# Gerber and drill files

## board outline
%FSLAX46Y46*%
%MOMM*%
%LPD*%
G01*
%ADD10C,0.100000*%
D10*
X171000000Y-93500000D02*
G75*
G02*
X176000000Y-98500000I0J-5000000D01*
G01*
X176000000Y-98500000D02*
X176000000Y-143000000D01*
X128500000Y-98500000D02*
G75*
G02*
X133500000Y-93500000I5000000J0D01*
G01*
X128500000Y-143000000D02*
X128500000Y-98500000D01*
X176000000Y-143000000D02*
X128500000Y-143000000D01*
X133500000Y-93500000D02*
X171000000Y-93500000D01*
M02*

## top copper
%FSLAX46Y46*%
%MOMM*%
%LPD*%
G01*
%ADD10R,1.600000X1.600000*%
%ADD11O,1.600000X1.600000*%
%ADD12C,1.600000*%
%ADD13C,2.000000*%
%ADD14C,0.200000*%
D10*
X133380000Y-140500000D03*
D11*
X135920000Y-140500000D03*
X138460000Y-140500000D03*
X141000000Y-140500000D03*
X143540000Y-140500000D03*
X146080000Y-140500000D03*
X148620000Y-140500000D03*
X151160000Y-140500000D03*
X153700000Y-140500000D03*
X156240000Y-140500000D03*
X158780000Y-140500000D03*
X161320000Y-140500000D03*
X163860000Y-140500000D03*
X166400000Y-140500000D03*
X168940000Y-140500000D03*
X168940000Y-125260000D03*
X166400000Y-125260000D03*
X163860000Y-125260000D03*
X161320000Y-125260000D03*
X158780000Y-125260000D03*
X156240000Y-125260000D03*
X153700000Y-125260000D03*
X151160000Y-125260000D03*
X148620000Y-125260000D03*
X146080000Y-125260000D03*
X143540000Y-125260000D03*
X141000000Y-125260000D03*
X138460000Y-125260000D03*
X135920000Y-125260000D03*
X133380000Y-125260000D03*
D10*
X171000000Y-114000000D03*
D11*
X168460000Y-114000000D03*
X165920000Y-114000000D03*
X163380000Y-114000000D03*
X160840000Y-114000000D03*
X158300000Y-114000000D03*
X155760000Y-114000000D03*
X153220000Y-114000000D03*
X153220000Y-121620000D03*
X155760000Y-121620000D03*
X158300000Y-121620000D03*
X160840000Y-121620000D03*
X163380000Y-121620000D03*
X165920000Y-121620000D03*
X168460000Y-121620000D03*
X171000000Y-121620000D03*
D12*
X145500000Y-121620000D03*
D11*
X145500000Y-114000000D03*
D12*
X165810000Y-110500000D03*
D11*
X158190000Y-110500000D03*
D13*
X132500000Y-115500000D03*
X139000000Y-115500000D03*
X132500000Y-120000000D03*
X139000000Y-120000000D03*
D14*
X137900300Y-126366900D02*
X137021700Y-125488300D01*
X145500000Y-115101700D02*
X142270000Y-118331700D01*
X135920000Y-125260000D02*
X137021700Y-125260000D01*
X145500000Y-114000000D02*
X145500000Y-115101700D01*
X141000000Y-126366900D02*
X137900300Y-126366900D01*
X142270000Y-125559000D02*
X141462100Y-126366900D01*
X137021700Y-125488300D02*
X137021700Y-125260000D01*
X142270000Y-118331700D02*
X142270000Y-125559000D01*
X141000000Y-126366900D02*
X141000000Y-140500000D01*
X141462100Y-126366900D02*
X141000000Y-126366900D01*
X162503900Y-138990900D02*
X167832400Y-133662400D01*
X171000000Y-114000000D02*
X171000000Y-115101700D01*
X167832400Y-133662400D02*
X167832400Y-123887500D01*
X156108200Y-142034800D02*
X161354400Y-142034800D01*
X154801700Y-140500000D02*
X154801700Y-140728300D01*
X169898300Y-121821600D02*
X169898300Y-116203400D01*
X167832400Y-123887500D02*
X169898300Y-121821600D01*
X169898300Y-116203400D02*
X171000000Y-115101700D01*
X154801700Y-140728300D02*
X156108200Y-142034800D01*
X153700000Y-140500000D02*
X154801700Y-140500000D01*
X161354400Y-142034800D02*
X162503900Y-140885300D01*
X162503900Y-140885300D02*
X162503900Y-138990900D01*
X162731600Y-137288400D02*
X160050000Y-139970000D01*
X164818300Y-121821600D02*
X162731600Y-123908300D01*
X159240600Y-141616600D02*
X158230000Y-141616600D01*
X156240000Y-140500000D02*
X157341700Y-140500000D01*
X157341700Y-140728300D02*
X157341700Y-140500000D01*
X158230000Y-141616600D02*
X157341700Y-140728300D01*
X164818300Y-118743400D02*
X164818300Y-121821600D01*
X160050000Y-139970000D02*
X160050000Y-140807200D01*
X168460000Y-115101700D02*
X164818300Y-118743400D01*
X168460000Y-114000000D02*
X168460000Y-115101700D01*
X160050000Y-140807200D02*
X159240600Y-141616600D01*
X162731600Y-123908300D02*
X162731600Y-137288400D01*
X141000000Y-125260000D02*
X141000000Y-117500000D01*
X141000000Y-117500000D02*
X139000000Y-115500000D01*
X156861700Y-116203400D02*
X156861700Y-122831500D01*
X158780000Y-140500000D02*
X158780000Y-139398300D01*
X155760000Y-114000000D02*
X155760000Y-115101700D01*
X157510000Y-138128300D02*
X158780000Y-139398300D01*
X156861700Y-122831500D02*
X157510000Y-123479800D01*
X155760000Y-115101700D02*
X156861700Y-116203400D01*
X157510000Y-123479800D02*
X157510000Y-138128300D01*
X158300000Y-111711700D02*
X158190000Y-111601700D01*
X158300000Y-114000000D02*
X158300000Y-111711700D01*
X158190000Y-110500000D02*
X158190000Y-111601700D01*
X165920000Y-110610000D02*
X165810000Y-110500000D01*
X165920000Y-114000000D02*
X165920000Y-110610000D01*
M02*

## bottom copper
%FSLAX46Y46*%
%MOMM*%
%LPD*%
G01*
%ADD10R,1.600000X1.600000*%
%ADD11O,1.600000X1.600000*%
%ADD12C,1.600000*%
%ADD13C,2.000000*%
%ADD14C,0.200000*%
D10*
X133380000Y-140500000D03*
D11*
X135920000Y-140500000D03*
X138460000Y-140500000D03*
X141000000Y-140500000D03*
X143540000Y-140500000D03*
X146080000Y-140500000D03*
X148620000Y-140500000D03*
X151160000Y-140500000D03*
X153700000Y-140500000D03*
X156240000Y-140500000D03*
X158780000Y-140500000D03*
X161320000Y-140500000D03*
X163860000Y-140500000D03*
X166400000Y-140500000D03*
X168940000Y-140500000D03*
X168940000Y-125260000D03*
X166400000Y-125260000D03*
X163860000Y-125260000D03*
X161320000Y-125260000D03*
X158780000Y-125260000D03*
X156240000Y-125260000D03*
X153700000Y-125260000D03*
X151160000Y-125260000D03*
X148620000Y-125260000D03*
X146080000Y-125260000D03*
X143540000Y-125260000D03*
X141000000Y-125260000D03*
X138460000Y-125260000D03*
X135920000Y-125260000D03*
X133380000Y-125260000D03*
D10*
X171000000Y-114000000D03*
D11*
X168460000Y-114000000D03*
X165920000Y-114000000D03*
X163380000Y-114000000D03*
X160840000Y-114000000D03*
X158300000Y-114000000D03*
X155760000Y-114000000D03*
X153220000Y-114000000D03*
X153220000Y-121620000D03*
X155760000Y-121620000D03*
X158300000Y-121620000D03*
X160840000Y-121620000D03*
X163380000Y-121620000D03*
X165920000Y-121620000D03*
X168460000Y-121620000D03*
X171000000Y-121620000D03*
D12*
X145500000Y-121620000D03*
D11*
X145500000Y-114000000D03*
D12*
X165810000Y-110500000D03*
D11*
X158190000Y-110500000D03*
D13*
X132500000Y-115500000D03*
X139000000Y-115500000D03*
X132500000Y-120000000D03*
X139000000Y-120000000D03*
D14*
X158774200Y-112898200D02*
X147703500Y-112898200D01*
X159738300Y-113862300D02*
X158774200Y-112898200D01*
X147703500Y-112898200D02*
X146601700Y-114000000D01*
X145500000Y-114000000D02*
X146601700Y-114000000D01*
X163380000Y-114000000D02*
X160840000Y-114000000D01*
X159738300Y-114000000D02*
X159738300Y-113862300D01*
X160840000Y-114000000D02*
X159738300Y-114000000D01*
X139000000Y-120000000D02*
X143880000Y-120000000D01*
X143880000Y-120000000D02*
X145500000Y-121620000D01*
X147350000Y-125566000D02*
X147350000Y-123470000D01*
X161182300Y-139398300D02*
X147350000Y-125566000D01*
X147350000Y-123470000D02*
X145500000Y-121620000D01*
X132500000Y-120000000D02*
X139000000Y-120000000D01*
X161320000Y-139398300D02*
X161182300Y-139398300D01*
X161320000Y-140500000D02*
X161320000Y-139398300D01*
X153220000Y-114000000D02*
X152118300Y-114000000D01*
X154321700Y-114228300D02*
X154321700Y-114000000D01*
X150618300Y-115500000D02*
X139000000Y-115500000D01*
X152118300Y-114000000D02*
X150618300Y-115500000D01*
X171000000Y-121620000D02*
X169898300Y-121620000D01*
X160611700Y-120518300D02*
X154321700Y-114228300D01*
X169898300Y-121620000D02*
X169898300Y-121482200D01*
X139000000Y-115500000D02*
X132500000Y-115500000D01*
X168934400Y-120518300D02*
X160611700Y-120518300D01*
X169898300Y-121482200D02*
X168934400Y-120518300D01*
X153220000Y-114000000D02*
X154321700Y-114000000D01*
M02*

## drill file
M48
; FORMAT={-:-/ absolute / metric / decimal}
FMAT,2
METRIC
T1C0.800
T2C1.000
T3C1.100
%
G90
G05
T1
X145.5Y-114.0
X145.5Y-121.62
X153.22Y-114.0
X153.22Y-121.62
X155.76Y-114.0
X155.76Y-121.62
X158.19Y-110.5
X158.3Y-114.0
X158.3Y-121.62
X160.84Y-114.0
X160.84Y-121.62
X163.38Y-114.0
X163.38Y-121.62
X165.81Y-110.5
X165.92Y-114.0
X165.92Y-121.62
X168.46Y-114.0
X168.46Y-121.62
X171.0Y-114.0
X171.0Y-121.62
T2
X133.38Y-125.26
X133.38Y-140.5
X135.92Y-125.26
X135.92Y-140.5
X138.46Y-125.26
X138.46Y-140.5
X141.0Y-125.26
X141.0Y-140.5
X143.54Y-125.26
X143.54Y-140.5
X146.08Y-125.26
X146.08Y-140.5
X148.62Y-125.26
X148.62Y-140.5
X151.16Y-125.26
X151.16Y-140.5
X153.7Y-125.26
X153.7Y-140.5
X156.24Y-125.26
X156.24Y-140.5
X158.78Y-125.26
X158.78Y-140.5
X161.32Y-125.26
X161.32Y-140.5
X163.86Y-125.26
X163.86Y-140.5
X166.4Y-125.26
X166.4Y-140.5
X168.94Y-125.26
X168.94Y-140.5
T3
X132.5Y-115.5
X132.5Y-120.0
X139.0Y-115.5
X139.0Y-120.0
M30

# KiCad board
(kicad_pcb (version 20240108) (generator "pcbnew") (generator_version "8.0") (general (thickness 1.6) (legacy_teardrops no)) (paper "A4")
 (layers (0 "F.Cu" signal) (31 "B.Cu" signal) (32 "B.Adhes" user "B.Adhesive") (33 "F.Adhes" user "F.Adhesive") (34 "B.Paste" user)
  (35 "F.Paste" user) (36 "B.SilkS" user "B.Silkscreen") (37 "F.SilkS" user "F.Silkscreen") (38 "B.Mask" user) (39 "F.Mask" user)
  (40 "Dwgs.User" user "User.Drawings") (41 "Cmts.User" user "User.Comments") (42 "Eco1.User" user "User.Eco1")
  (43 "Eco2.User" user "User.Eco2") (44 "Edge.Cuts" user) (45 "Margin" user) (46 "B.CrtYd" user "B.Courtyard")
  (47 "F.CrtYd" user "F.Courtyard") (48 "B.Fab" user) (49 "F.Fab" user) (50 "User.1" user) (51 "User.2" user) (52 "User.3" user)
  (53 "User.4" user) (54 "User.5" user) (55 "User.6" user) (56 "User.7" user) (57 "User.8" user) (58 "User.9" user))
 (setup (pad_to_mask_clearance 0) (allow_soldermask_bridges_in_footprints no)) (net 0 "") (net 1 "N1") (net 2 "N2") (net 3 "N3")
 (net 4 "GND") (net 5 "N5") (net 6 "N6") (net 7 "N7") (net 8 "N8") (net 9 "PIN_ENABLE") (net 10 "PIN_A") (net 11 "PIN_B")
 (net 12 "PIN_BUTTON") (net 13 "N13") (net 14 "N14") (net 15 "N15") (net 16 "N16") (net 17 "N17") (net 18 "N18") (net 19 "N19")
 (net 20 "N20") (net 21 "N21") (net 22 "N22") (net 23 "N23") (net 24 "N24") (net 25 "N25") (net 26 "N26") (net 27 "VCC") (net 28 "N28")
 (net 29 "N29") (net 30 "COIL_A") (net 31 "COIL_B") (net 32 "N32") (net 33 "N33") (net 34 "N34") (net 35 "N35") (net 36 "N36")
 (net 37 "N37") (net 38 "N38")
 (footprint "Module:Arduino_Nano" (layer "F.Cu") (at 133.38 140.5 90)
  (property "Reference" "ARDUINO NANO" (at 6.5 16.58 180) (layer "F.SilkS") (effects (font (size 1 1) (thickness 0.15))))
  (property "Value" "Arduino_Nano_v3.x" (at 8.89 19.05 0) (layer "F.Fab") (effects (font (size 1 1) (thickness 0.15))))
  (pad "1" thru_hole rect (at 0 0 90) (size 1.6 1.6) (drill 1) (layers "*.Cu" "*.Mask") (remove_unused_layers no) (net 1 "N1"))
  (pad "2" thru_hole oval (at 0 2.54 90) (size 1.6 1.6) (drill 1) (layers "*.Cu" "*.Mask") (remove_unused_layers no) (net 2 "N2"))
  (pad "3" thru_hole oval (at 0 5.08 90) (size 1.6 1.6) (drill 1) (layers "*.Cu" "*.Mask") (remove_unused_layers no) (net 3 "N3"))
  (pad "4" thru_hole oval (at 0 7.62 90) (size 1.6 1.6) (drill 1) (layers "*.Cu" "*.Mask") (remove_unused_layers no) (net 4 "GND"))
  (pad "5" thru_hole oval (at 0 10.16 90) (size 1.6 1.6) (drill 1) (layers "*.Cu" "*.Mask") (remove_unused_layers no) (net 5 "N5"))
  (pad "6" thru_hole oval (at 0 12.7 90) (size 1.6 1.6) (drill 1) (layers "*.Cu" "*.Mask") (remove_unused_layers no) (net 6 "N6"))
  (pad "7" thru_hole oval (at 0 15.24 90) (size 1.6 1.6) (drill 1) (layers "*.Cu" "*.Mask") (remove_unused_layers no) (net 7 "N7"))
  (pad "8" thru_hole oval (at 0 17.78 90) (size 1.6 1.6) (drill 1) (layers "*.Cu" "*.Mask") (remove_unused_layers no) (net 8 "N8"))
  (pad "9" thru_hole oval (at 0 20.32 90) (size 1.6 1.6) (drill 1) (layers "*.Cu" "*.Mask") (remove_unused_layers no) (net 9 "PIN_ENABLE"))
  (pad "10" thru_hole oval (at 0 22.86 90) (size 1.6 1.6) (drill 1) (layers "*.Cu" "*.Mask") (remove_unused_layers no) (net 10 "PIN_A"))
  (pad "11" thru_hole oval (at 0 25.4 90) (size 1.6 1.6) (drill 1) (layers "*.Cu" "*.Mask") (remove_unused_layers no) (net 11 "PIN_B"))
  (pad "12" thru_hole oval (at 0 27.94 90) (size 1.6 1.6) (drill 1) (layers "*.Cu" "*.Mask") (remove_unused_layers no) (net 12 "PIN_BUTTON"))
  (pad "13" thru_hole oval (at 0 30.48 90) (size 1.6 1.6) (drill 1) (layers "*.Cu" "*.Mask") (remove_unused_layers no) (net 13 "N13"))
  (pad "14" thru_hole oval (at 0 33.02 90) (size 1.6 1.6) (drill 1) (layers "*.Cu" "*.Mask") (remove_unused_layers no) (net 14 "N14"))
  (pad "15" thru_hole oval (at 0 35.56 90) (size 1.6 1.6) (drill 1) (layers "*.Cu" "*.Mask") (remove_unused_layers no) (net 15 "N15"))
  (pad "16" thru_hole oval (at 15.24 35.56 90) (size 1.6 1.6) (drill 1) (layers "*.Cu" "*.Mask") (remove_unused_layers no) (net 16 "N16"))
  (pad "17" thru_hole oval (at 15.24 33.02 90) (size 1.6 1.6) (drill 1) (layers "*.Cu" "*.Mask") (remove_unused_layers no) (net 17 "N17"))
  (pad "18" thru_hole oval (at 15.24 30.48 90) (size 1.6 1.6) (drill 1) (layers "*.Cu" "*.Mask") (remove_unused_layers no) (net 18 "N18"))
  (pad "19" thru_hole oval (at 15.24 27.94 90) (size 1.6 1.6) (drill 1) (layers "*.Cu" "*.Mask") (remove_unused_layers no) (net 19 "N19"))
  (pad "20" thru_hole oval (at 15.24 25.4 90) (size 1.6 1.6) (drill 1) (layers "*.Cu" "*.Mask") (remove_unused_layers no) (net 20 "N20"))
  (pad "21" thru_hole oval (at 15.24 22.86 90) (size 1.6 1.6) (drill 1) (layers "*.Cu" "*.Mask") (remove_unused_layers no) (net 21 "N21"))
  (pad "22" thru_hole oval (at 15.24 20.32 90) (size 1.6 1.6) (drill 1) (layers "*.Cu" "*.Mask") (remove_unused_layers no) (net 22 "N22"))
  (pad "23" thru_hole oval (at 15.24 17.78 90) (size 1.6 1.6) (drill 1) (layers "*.Cu" "*.Mask") (remove_unused_layers no) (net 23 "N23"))
  (pad "24" thru_hole oval (at 15.24 15.24 90) (size 1.6 1.6) (drill 1) (layers "*.Cu" "*.Mask") (remove_unused_layers no) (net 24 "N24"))
  (pad "25" thru_hole oval (at 15.24 12.7 90) (size 1.6 1.6) (drill 1) (layers "*.Cu" "*.Mask") (remove_unused_layers no) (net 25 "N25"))
  (pad "26" thru_hole oval (at 15.24 10.16 90) (size 1.6 1.6) (drill 1) (layers "*.Cu" "*.Mask") (remove_unused_layers no) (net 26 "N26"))
  (pad "27" thru_hole oval (at 15.24 7.62 90) (size 1.6 1.6) (drill 1) (layers "*.Cu" "*.Mask") (remove_unused_layers no) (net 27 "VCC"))
  (pad "28" thru_hole oval (at 15.24 5.08 90) (size 1.6 1.6) (drill 1) (layers "*.Cu" "*.Mask") (remove_unused_layers no) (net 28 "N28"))
  (pad "29" thru_hole oval (at 15.24 2.54 90) (size 1.6 1.6) (drill 1) (layers "*.Cu" "*.Mask") (remove_unused_layers no) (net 4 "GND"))
  (pad "30" thru_hole oval (at 15.24 0 90) (size 1.6 1.6) (drill 1) (layers "*.Cu" "*.Mask") (remove_unused_layers no) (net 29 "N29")))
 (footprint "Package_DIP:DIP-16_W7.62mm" (layer "F.Cu") (at 171 114 -90)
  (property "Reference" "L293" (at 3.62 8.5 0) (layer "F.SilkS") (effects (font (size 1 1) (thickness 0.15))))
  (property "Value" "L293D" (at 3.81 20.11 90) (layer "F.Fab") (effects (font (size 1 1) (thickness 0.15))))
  (pad "1" thru_hole rect (at 0 0 270) (size 1.6 1.6) (drill 0.8) (layers "*.Cu" "*.Mask") (remove_unused_layers no) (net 9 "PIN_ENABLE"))
  (pad "2" thru_hole oval (at 0 2.54 270) (size 1.6 1.6) (drill 0.8) (layers "*.Cu" "*.Mask") (remove_unused_layers no) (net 10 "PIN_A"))
  (pad "3" thru_hole oval (at 0 5.08 270) (size 1.6 1.6) (drill 0.8) (layers "*.Cu" "*.Mask") (remove_unused_layers no) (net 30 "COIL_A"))
  (pad "4" thru_hole oval (at 0 7.62 270) (size 1.6 1.6) (drill 0.8) (layers "*.Cu" "*.Mask") (remove_unused_layers no) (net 4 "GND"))
  (pad "5" thru_hole oval (at 0 10.16 270) (size 1.6 1.6) (drill 0.8) (layers "*.Cu" "*.Mask") (remove_unused_layers no) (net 4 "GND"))
  (pad "6" thru_hole oval (at 0 12.7 270) (size 1.6 1.6) (drill 0.8) (layers "*.Cu" "*.Mask") (remove_unused_layers no) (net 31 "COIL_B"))
  (pad "7" thru_hole oval (at 0 15.24 270) (size 1.6 1.6) (drill 0.8) (layers "*.Cu" "*.Mask") (remove_unused_layers no) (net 11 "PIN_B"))
  (pad "8" thru_hole oval (at 0 17.78 270) (size 1.6 1.6) (drill 0.8) (layers "*.Cu" "*.Mask") (remove_unused_layers no) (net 27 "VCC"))
  (pad "9" thru_hole oval (at 7.62 17.78 270) (size 1.6 1.6) (drill 0.8) (layers "*.Cu" "*.Mask") (remove_unused_layers no) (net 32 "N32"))
  (pad "10" thru_hole oval (at 7.62 15.24 270) (size 1.6 1.6) (drill 0.8) (layers "*.Cu" "*.Mask") (remove_unused_layers no) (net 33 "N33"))
  (pad "11" thru_hole oval (at 7.62 12.7 270) (size 1.6 1.6) (drill 0.8) (layers "*.Cu" "*.Mask") (remove_unused_layers no) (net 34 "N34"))
  (pad "12" thru_hole oval (at 7.62 10.16 270) (size 1.6 1.6) (drill 0.8) (layers "*.Cu" "*.Mask") (remove_unused_layers no) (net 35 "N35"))
  (pad "13" thru_hole oval (at 7.62 7.62 270) (size 1.6 1.6) (drill 0.8) (layers "*.Cu" "*.Mask") (remove_unused_layers no) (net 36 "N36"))
  (pad "14" thru_hole oval (at 7.62 5.08 270) (size 1.6 1.6) (drill 0.8) (layers "*.Cu" "*.Mask") (remove_unused_layers no) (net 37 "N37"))
  (pad "15" thru_hole oval (at 7.62 2.54 270) (size 1.6 1.6) (drill 0.8) (layers "*.Cu" "*.Mask") (remove_unused_layers no) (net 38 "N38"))
  (pad "16" thru_hole oval (at 7.62 0 270) (size 1.6 1.6) (drill 0.8) (layers "*.Cu" "*.Mask") (remove_unused_layers no) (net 27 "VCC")))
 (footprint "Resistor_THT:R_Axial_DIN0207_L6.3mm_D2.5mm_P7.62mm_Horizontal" (layer "F.Cu") (at 145.5 121.62 90)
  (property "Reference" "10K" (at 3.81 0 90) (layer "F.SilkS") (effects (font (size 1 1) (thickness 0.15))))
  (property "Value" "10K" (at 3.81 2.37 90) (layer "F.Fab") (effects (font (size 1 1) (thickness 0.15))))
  (pad "1" thru_hole circle (at 0 0 90) (size 1.6 1.6) (drill 0.8) (layers "*.Cu" "*.Mask") (remove_unused_layers no) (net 12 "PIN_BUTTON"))
  (pad "2" thru_hole oval (at 7.62 0 90) (size 1.6 1.6) (drill 0.8) (layers "*.Cu" "*.Mask") (remove_unused_layers no) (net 4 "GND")))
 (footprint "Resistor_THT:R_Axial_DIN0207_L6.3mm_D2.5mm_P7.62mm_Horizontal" (layer "F.Cu") (at 165.81 110.5 180)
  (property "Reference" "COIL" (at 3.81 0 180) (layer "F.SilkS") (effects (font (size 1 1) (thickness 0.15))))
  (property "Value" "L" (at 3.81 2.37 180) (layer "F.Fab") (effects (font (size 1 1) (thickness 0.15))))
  (pad "1" thru_hole circle (at 0 0 180) (size 1.6 1.6) (drill 0.8) (layers "*.Cu" "*.Mask") (remove_unused_layers no) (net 30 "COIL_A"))
  (pad "2" thru_hole oval (at 7.62 0 180) (size 1.6 1.6) (drill 0.8) (layers "*.Cu" "*.Mask") (remove_unused_layers no) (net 31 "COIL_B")))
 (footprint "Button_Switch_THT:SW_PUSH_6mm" (layer "F.Cu") (at 132.5 115.5)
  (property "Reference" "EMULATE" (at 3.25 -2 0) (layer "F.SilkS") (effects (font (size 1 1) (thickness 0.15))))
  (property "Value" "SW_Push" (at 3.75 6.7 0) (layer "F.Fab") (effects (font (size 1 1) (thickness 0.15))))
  (pad "1" thru_hole circle (at 0 0 90) (size 2 2) (drill 1.1) (layers "*.Cu" "*.Mask") (remove_unused_layers no) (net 27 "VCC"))
  (pad "1" thru_hole circle (at 6.5 0 90) (size 2 2) (drill 1.1) (layers "*.Cu" "*.Mask") (remove_unused_layers no) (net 27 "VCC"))
  (pad "2" thru_hole circle (at 0 4.5 90) (size 2 2) (drill 1.1) (layers "*.Cu" "*.Mask") (remove_unused_layers no) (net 12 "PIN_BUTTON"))
  (pad "2" thru_hole circle (at 6.5 4.5 90) (size 2 2) (drill 1.1) (layers "*.Cu" "*.Mask") (remove_unused_layers no) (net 12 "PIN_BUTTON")))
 (gr_arc (start 171 93.5) (mid 174.535534 94.964466) (end 176 98.5) (stroke (width 0.1) (type default)) (layer "Edge.Cuts"))
 (gr_line (start 176 98.5) (end 176 143) (stroke (width 0.1) (type default)) (layer "Edge.Cuts"))
 (gr_arc (start 128.5 98.5) (mid 129.964466 94.964466) (end 133.5 93.5) (stroke (width 0.1) (type default)) (layer "Edge.Cuts"))
 (gr_line (start 128.5 143) (end 128.5 98.5) (stroke (width 0.1) (type default)) (layer "Edge.Cuts"))
 (gr_line (start 176 143) (end 128.5 143) (stroke (width 0.1) (type default)) (layer "Edge.Cuts"))
 (gr_line (start 133.5 93.5) (end 171 93.5) (stroke (width 0.1) (type default)) (layer "Edge.Cuts"))
 (segment (start 137.9003 126.3669) (end 137.0217 125.4883) (width 0.2) (layer "F.Cu") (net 4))
 (segment (start 145.5 115.1017) (end 142.27 118.3317) (width 0.2) (layer "F.Cu") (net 4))
 (segment (start 135.92 125.26) (end 137.0217 125.26) (width 0.2) (layer "F.Cu") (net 4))
 (segment (start 145.5 114) (end 145.5 115.1017) (width 0.2) (layer "F.Cu") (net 4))
 (segment (start 141 126.3669) (end 137.9003 126.3669) (width 0.2) (layer "F.Cu") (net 4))
 (segment (start 142.27 125.559) (end 141.4621 126.3669) (width 0.2) (layer "F.Cu") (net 4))
 (segment (start 137.0217 125.4883) (end 137.0217 125.26) (width 0.2) (layer "F.Cu") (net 4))
 (segment (start 142.27 118.3317) (end 142.27 125.559) (width 0.2) (layer "F.Cu") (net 4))
 (segment (start 141 126.3669) (end 141 140.5) (width 0.2) (layer "F.Cu") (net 4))
 (segment (start 141.4621 126.3669) (end 141 126.3669) (width 0.2) (layer "F.Cu") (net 4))
 (segment (start 158.7742 112.8982) (end 147.7035 112.8982) (width 0.2) (layer "B.Cu") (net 4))
 (segment (start 159.7383 113.8623) (end 158.7742 112.8982) (width 0.2) (layer "B.Cu") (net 4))
 (segment (start 147.7035 112.8982) (end 146.6017 114) (width 0.2) (layer "B.Cu") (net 4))
 (segment (start 145.5 114) (end 146.6017 114) (width 0.2) (layer "B.Cu") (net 4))
 (segment (start 163.38 114) (end 160.84 114) (width 0.2) (layer "B.Cu") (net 4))
 (segment (start 159.7383 114) (end 159.7383 113.8623) (width 0.2) (layer "B.Cu") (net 4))
 (segment (start 160.84 114) (end 159.7383 114) (width 0.2) (layer "B.Cu") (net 4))
 (segment (start 139 120) (end 143.88 120) (width 0.2) (layer "B.Cu") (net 12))
 (segment (start 143.88 120) (end 145.5 121.62) (width 0.2) (layer "B.Cu") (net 12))
 (segment (start 147.35 125.566) (end 147.35 123.47) (width 0.2) (layer "B.Cu") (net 12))
 (segment (start 161.1823 139.3983) (end 147.35 125.566) (width 0.2) (layer "B.Cu") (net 12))
 (segment (start 147.35 123.47) (end 145.5 121.62) (width 0.2) (layer "B.Cu") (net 12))
 (segment (start 132.5 120) (end 139 120) (width 0.2) (layer "B.Cu") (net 12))
 (segment (start 161.32 139.3983) (end 161.1823 139.3983) (width 0.2) (layer "B.Cu") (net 12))
 (segment (start 161.32 140.5) (end 161.32 139.3983) (width 0.2) (layer "B.Cu") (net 12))
 (segment (start 162.5039 138.9909) (end 167.8324 133.6624) (width 0.2) (layer "F.Cu") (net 9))
 (segment (start 171 114) (end 171 115.1017) (width 0.2) (layer "F.Cu") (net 9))
 (segment (start 167.8324 133.6624) (end 167.8324 123.8875) (width 0.2) (layer "F.Cu") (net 9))
 (segment (start 156.1082 142.0348) (end 161.3544 142.0348) (width 0.2) (layer "F.Cu") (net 9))
 (segment (start 154.8017 140.5) (end 154.8017 140.7283) (width 0.2) (layer "F.Cu") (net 9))
 (segment (start 169.8983 121.8216) (end 169.8983 116.2034) (width 0.2) (layer "F.Cu") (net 9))
 (segment (start 167.8324 123.8875) (end 169.8983 121.8216) (width 0.2) (layer "F.Cu") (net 9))
 (segment (start 169.8983 116.2034) (end 171 115.1017) (width 0.2) (layer "F.Cu") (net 9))
 (segment (start 154.8017 140.7283) (end 156.1082 142.0348) (width 0.2) (layer "F.Cu") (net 9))
 (segment (start 153.7 140.5) (end 154.8017 140.5) (width 0.2) (layer "F.Cu") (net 9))
 (segment (start 161.3544 142.0348) (end 162.5039 140.8853) (width 0.2) (layer "F.Cu") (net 9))
 (segment (start 162.5039 140.8853) (end 162.5039 138.9909) (width 0.2) (layer "F.Cu") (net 9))
 (segment (start 162.7316 137.2884) (end 160.05 139.97) (width 0.2) (layer "F.Cu") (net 10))
 (segment (start 164.8183 121.8216) (end 162.7316 123.9083) (width 0.2) (layer "F.Cu") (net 10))
 (segment (start 159.2406 141.6166) (end 158.23 141.6166) (width 0.2) (layer "F.Cu") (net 10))
 (segment (start 156.24 140.5) (end 157.3417 140.5) (width 0.2) (layer "F.Cu") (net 10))
 (segment (start 157.3417 140.7283) (end 157.3417 140.5) (width 0.2) (layer "F.Cu") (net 10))
 (segment (start 158.23 141.6166) (end 157.3417 140.7283) (width 0.2) (layer "F.Cu") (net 10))
 (segment (start 164.8183 118.7434) (end 164.8183 121.8216) (width 0.2) (layer "F.Cu") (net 10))
 (segment (start 160.05 139.97) (end 160.05 140.8072) (width 0.2) (layer "F.Cu") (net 10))
 (segment (start 168.46 115.1017) (end 164.8183 118.7434) (width 0.2) (layer "F.Cu") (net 10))
 (segment (start 168.46 114) (end 168.46 115.1017) (width 0.2) (layer "F.Cu") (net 10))
 (segment (start 160.05 140.8072) (end 159.2406 141.6166) (width 0.2) (layer "F.Cu") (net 10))
 (segment (start 162.7316 123.9083) (end 162.7316 137.2884) (width 0.2) (layer "F.Cu") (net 10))
 (segment (start 141 125.26) (end 141 117.5) (width 0.2) (layer "F.Cu") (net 27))
 (segment (start 141 117.5) (end 139 115.5) (width 0.2) (layer "F.Cu") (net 27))
 (segment (start 153.22 114) (end 152.1183 114) (width 0.2) (layer "B.Cu") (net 27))
 (segment (start 154.3217 114.2283) (end 154.3217 114) (width 0.2) (layer "B.Cu") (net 27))
 (segment (start 150.6183 115.5) (end 139 115.5) (width 0.2) (layer "B.Cu") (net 27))
 (segment (start 152.1183 114) (end 150.6183 115.5) (width 0.2) (layer "B.Cu") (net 27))
 (segment (start 171 121.62) (end 169.8983 121.62) (width 0.2) (layer "B.Cu") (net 27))
 (segment (start 160.6117 120.5183) (end 154.3217 114.2283) (width 0.2) (layer "B.Cu") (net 27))
 (segment (start 169.8983 121.62) (end 169.8983 121.4822) (width 0.2) (layer "B.Cu") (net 27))
 (segment (start 139 115.5) (end 132.5 115.5) (width 0.2) (layer "B.Cu") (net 27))
 (segment (start 168.9344 120.5183) (end 160.6117 120.5183) (width 0.2) (layer "B.Cu") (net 27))
 (segment (start 169.8983 121.4822) (end 168.9344 120.5183) (width 0.2) (layer "B.Cu") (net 27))
 (segment (start 153.22 114) (end 154.3217 114) (width 0.2) (layer "B.Cu") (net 27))
 (segment (start 156.8617 116.2034) (end 156.8617 122.8315) (width 0.2) (layer "F.Cu") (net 11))
 (segment (start 158.78 140.5) (end 158.78 139.3983) (width 0.2) (layer "F.Cu") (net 11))
 (segment (start 155.76 114) (end 155.76 115.1017) (width 0.2) (layer "F.Cu") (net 11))
 (segment (start 157.51 138.1283) (end 158.78 139.3983) (width 0.2) (layer "F.Cu") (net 11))
 (segment (start 156.8617 122.8315) (end 157.51 123.4798) (width 0.2) (layer "F.Cu") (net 11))
 (segment (start 155.76 115.1017) (end 156.8617 116.2034) (width 0.2) (layer "F.Cu") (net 11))
 (segment (start 157.51 123.4798) (end 157.51 138.1283) (width 0.2) (layer "F.Cu") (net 11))
 (segment (start 158.3 111.7117) (end 158.19 111.6017) (width 0.2) (layer "F.Cu") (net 31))
 (segment (start 158.3 114) (end 158.3 111.7117) (width 0.2) (layer "F.Cu") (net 31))
 (segment (start 158.19 110.5) (end 158.19 111.6017) (width 0.2) (layer "F.Cu") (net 31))
 (segment (start 165.92 110.61) (end 165.81 110.5) (width 0.2) (layer "F.Cu") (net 30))
 (segment (start 165.92 114) (end 165.92 110.61) (width 0.2) (layer "F.Cu") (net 30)))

